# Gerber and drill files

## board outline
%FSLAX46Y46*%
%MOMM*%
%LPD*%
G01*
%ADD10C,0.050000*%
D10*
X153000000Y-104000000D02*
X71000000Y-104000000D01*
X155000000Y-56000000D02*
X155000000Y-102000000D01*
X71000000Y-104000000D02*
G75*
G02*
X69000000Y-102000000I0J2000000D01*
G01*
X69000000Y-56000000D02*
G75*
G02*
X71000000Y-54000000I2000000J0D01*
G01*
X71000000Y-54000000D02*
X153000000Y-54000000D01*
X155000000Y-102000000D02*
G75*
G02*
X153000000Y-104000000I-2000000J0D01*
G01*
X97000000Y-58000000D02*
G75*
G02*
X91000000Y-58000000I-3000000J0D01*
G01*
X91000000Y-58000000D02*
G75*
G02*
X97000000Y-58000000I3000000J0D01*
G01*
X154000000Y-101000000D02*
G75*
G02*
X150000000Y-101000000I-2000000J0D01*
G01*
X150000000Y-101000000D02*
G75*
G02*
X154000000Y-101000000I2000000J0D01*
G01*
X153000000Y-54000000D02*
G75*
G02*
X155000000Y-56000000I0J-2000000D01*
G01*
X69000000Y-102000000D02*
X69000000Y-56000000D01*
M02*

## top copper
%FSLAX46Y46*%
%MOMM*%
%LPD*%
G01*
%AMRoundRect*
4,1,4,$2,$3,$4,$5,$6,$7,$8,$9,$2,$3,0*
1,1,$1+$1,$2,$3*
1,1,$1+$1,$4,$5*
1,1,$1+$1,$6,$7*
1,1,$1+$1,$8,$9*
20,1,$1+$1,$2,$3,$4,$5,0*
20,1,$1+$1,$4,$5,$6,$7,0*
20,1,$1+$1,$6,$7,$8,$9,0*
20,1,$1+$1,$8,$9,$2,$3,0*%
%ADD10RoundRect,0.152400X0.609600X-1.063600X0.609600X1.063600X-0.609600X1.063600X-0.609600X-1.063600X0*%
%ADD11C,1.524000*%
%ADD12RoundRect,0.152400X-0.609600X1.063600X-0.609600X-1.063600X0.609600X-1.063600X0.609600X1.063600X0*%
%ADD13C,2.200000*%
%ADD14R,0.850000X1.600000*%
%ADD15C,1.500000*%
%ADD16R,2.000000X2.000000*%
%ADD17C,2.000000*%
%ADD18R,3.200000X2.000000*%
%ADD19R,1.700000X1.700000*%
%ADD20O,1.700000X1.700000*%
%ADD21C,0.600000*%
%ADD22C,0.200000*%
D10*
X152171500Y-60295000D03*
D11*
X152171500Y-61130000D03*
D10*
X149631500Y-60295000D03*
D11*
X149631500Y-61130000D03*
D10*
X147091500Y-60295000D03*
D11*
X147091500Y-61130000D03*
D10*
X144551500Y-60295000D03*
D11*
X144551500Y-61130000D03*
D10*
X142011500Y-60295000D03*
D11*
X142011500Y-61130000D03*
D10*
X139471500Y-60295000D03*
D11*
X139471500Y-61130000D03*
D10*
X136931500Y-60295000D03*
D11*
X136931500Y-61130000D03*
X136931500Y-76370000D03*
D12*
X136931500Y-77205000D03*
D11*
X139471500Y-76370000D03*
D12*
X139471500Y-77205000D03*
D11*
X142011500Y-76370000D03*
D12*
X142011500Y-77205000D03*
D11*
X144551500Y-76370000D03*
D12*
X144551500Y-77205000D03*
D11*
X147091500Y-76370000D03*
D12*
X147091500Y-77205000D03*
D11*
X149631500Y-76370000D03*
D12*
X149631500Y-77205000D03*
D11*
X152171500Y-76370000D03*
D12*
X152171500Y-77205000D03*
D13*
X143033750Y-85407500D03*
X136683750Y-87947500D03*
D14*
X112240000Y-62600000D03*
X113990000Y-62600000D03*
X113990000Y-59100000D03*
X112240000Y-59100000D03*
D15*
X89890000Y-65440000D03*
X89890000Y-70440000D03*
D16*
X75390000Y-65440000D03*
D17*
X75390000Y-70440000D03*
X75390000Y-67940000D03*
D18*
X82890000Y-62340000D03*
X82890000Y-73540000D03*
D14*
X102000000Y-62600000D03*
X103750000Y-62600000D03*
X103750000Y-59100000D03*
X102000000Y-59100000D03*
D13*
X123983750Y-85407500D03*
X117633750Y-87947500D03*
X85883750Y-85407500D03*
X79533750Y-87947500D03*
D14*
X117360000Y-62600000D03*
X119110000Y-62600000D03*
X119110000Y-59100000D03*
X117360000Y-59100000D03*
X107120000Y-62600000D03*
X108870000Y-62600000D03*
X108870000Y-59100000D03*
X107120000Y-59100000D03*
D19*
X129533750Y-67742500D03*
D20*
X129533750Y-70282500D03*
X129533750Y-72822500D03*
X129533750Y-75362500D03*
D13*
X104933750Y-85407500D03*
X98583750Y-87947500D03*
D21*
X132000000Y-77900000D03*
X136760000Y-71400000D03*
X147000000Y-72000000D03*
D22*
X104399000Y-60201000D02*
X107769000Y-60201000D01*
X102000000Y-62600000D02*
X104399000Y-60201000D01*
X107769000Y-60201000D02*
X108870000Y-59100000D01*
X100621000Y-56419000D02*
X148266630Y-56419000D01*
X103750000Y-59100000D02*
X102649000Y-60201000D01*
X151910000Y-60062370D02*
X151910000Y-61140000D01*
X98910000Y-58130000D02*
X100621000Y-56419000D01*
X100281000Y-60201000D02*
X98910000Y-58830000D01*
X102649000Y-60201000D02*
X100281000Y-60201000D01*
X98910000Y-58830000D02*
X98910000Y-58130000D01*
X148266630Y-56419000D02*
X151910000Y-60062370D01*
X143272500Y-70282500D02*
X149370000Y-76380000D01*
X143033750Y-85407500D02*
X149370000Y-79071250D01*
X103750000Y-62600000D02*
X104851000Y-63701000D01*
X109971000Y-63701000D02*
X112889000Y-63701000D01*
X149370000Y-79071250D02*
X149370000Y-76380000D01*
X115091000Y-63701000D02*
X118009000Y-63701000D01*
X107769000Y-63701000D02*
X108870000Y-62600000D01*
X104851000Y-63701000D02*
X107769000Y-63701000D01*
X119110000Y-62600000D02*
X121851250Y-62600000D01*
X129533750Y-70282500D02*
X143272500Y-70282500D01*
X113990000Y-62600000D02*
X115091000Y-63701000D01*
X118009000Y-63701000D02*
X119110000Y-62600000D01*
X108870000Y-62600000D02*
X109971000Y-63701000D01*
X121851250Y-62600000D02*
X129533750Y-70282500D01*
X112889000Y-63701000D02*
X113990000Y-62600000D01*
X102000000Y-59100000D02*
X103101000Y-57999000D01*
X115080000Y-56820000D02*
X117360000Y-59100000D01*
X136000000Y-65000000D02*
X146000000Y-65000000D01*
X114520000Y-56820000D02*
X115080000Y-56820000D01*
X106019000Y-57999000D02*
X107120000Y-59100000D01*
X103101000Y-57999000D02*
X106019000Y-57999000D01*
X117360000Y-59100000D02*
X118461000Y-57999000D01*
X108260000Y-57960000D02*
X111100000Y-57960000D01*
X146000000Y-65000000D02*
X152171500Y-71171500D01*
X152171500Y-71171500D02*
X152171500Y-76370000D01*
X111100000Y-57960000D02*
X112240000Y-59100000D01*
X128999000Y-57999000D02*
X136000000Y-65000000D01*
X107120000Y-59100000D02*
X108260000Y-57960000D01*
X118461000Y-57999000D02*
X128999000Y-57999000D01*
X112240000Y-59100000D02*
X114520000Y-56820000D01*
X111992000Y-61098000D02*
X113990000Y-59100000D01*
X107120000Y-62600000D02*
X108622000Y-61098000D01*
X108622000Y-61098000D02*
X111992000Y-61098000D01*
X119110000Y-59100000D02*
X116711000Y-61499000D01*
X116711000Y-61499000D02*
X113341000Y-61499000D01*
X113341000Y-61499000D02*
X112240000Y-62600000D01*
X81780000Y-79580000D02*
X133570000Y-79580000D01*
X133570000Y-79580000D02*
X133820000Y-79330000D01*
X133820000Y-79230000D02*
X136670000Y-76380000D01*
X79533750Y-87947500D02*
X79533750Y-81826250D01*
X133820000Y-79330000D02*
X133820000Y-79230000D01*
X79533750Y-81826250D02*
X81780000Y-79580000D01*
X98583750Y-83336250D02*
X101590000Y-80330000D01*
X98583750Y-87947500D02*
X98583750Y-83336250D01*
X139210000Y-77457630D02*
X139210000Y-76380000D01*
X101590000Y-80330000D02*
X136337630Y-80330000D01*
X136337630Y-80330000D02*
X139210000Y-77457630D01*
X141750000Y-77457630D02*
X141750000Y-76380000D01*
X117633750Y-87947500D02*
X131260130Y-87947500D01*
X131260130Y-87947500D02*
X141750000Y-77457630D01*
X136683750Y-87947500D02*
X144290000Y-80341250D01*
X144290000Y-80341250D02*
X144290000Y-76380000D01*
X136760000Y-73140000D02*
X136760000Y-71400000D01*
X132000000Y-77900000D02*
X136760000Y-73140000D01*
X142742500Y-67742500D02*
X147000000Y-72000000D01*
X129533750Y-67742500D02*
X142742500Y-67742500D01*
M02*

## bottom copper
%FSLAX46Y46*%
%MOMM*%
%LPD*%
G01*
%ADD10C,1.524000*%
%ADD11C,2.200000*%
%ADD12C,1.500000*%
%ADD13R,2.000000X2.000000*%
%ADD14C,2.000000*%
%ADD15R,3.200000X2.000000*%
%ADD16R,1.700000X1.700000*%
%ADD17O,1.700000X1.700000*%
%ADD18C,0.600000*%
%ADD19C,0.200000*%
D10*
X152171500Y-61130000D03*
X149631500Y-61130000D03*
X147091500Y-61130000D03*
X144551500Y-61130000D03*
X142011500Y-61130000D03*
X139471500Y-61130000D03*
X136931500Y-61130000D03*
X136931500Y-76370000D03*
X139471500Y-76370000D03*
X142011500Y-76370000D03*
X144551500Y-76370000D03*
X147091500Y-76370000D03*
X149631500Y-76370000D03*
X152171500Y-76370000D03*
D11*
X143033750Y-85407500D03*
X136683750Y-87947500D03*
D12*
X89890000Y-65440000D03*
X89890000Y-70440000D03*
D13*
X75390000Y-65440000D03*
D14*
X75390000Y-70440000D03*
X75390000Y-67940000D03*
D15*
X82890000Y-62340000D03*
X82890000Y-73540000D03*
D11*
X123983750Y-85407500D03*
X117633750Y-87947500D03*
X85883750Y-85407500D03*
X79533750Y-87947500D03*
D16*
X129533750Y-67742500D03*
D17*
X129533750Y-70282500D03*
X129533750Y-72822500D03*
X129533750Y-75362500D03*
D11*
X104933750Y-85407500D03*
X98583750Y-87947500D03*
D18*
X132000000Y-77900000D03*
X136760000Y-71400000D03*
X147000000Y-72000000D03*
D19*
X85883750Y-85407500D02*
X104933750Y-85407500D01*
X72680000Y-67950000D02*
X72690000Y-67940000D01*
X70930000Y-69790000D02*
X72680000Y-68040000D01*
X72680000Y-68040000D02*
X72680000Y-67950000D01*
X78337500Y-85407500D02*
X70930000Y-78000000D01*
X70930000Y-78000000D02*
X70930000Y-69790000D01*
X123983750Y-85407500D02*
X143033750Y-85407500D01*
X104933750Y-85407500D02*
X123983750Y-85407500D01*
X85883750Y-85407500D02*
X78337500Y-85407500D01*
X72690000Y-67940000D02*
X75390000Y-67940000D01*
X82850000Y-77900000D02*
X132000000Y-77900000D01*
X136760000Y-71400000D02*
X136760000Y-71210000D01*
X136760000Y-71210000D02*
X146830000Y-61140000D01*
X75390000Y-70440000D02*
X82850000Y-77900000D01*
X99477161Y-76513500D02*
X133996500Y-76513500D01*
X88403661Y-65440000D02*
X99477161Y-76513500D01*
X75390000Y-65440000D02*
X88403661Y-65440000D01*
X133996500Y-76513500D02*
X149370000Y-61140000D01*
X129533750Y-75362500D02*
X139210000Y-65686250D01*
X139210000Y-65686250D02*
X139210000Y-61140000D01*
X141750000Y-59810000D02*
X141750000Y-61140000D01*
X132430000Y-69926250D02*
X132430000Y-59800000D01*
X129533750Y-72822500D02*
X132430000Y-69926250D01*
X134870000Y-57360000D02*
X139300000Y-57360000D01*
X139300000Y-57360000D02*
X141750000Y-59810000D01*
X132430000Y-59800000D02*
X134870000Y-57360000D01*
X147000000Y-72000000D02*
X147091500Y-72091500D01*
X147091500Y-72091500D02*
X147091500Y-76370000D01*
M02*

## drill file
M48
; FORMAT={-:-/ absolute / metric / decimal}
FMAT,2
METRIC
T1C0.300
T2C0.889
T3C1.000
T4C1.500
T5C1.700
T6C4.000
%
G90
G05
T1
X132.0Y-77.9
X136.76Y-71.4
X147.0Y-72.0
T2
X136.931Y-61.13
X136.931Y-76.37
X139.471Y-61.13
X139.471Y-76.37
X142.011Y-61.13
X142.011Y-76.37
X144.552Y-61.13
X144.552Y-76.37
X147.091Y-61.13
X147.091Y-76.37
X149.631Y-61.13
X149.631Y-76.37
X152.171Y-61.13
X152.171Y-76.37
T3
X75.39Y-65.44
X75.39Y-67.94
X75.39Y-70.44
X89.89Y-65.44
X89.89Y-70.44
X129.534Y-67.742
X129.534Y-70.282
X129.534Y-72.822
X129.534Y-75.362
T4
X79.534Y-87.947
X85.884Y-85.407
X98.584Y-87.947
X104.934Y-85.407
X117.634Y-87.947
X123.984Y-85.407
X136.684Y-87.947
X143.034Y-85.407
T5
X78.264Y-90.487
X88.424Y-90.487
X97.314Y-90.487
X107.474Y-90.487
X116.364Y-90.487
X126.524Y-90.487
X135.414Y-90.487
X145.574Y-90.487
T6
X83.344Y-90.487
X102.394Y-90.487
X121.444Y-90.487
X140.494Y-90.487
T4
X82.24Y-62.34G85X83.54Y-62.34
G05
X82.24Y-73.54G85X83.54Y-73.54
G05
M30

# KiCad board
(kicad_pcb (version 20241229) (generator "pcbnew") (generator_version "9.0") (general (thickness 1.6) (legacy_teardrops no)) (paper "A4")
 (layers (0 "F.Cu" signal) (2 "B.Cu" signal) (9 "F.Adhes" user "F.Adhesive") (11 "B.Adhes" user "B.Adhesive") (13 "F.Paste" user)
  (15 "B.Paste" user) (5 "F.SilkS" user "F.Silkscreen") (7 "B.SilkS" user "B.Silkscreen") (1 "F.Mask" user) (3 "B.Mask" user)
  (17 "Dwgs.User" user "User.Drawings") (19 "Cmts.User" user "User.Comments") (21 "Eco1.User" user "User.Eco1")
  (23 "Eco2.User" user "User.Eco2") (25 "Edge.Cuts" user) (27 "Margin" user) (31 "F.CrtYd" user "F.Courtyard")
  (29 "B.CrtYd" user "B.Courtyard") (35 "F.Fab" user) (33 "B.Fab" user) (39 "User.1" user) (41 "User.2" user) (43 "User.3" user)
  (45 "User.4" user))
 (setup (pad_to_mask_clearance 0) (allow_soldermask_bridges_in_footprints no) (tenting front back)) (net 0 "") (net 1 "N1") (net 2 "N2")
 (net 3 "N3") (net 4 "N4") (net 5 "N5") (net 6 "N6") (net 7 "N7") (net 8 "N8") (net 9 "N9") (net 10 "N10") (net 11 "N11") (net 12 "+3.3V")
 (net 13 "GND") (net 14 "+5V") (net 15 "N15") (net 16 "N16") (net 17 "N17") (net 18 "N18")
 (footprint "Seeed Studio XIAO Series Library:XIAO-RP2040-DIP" (layer "F.Cu") (at 144.5515 68.75 -90)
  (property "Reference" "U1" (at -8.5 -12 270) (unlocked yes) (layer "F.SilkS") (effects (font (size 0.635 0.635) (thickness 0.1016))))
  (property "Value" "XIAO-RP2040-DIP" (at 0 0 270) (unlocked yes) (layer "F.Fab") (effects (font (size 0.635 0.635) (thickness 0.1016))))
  (pad "1" smd roundrect (at -8.455 -7.62 90) (size 2.432 1.524) (layers "F.Cu" "F.Mask") (roundrect_rratio 0.1) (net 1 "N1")
   (thermal_bridge_angle 45))
  (pad "1" thru_hole circle (at -7.62 -7.62 90) (size 1.524 1.524) (drill 0.889) (layers "*.Cu" "*.Mask") (remove_unused_layers no)
   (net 1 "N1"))
  (pad "2" smd roundrect (at -8.455 -5.08 90) (size 2.432 1.524) (layers "F.Cu" "F.Mask") (roundrect_rratio 0.1) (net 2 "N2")
   (thermal_bridge_angle 45))
  (pad "2" thru_hole circle (at -7.62 -5.08 90) (size 1.524 1.524) (drill 0.889) (layers "*.Cu" "*.Mask") (remove_unused_layers no)
   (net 2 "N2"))
  (pad "3" smd roundrect (at -8.455 -2.54 90) (size 2.432 1.524) (layers "F.Cu" "F.Mask") (roundrect_rratio 0.1) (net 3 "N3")
   (thermal_bridge_angle 45))
  (pad "3" thru_hole circle (at -7.62 -2.54 90) (size 1.524 1.524) (drill 0.889) (layers "*.Cu" "*.Mask") (remove_unused_layers no)
   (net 3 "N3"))
  (pad "4" smd roundrect (at -8.455 0 90) (size 2.432 1.524) (layers "F.Cu" "F.Mask") (roundrect_rratio 0.1) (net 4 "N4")
   (thermal_bridge_angle 45))
  (pad "4" thru_hole circle (at -7.62 0 90) (size 1.524 1.524) (drill 0.889) (layers "*.Cu" "*.Mask") (remove_unused_layers no) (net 4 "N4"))
  (pad "5" smd roundrect (at -8.455 2.54 90) (size 2.432 1.524) (layers "F.Cu" "F.Mask") (roundrect_rratio 0.1) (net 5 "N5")
   (thermal_bridge_angle 45))
  (pad "5" thru_hole circle (at -7.62 2.54 90) (size 1.524 1.524) (drill 0.889) (layers "*.Cu" "*.Mask") (remove_unused_layers no)
   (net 5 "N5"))
  (pad "6" smd roundrect (at -8.455 5.08 90) (size 2.432 1.524) (layers "F.Cu" "F.Mask") (roundrect_rratio 0.1) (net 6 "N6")
   (thermal_bridge_angle 45))
  (pad "6" thru_hole circle (at -7.62 5.08 90) (size 1.524 1.524) (drill 0.889) (layers "*.Cu" "*.Mask") (remove_unused_layers no)
   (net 6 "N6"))
  (pad "7" smd roundrect (at -8.455 7.62 90) (size 2.432 1.524) (layers "F.Cu" "F.Mask") (roundrect_rratio 0.1) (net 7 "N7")
   (thermal_bridge_angle 45))
  (pad "7" thru_hole circle (at -7.62 7.62 90) (size 1.524 1.524) (drill 0.889) (layers "*.Cu" "*.Mask") (remove_unused_layers no)
   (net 7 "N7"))
  (pad "8" thru_hole circle (at 7.62 7.62 270) (size 1.524 1.524) (drill 0.889) (layers "*.Cu" "*.Mask") (remove_unused_layers no)
   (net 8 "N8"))
  (pad "8" smd roundrect (at 8.455 7.62 270) (size 2.432 1.524) (layers "F.Cu" "F.Mask") (roundrect_rratio 0.1) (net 8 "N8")
   (thermal_bridge_angle 45))
  (pad "9" thru_hole circle (at 7.62 5.08 270) (size 1.524 1.524) (drill 0.889) (layers "*.Cu" "*.Mask") (remove_unused_layers no)
   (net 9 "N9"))
  (pad "9" smd roundrect (at 8.455 5.08 270) (size 2.432 1.524) (layers "F.Cu" "F.Mask") (roundrect_rratio 0.1) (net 9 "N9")
   (thermal_bridge_angle 45))
  (pad "10" thru_hole circle (at 7.62 2.54 270) (size 1.524 1.524) (drill 0.889) (layers "*.Cu" "*.Mask") (remove_unused_layers no)
   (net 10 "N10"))
  (pad "10" smd roundrect (at 8.455 2.54 270) (size 2.432 1.524) (layers "F.Cu" "F.Mask") (roundrect_rratio 0.1) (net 10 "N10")
   (thermal_bridge_angle 45))
  (pad "11" thru_hole circle (at 7.62 0 270) (size 1.524 1.524) (drill 0.889) (layers "*.Cu" "*.Mask") (remove_unused_layers no)
   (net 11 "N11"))
  (pad "11" smd roundrect (at 8.455 0 270) (size 2.432 1.524) (layers "F.Cu" "F.Mask") (roundrect_rratio 0.1) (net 11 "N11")
   (thermal_bridge_angle 45))
  (pad "12" thru_hole circle (at 7.62 -2.54 270) (size 1.524 1.524) (drill 0.889) (layers "*.Cu" "*.Mask") (remove_unused_layers no)
   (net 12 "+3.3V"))
  (pad "12" smd roundrect (at 8.455 -2.54 270) (size 2.432 1.524) (layers "F.Cu" "F.Mask") (roundrect_rratio 0.1) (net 12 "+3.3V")
   (thermal_bridge_angle 45))
  (pad "13" thru_hole circle (at 7.62 -5.08 270) (size 1.524 1.524) (drill 0.889) (layers "*.Cu" "*.Mask") (remove_unused_layers no)
   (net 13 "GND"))
  (pad "13" smd roundrect (at 8.455 -5.08 270) (size 2.432 1.524) (layers "F.Cu" "F.Mask") (roundrect_rratio 0.1) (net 13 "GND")
   (thermal_bridge_angle 45))
  (pad "14" thru_hole circle (at 7.62 -7.62 270) (size 1.524 1.524) (drill 0.889) (layers "*.Cu" "*.Mask") (remove_unused_layers no)
   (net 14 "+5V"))
  (pad "14" smd roundrect (at 8.455 -7.62 270) (size 2.432 1.524) (layers "F.Cu" "F.Mask") (roundrect_rratio 0.1) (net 14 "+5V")
   (thermal_bridge_angle 45)))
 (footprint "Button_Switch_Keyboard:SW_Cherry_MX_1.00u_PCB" (layer "F.Cu") (at 143.03375 85.4075)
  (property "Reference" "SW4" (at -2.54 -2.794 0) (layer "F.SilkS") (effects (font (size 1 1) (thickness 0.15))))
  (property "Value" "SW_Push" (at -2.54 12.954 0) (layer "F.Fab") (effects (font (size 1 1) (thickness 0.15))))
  (pad "" np_thru_hole circle (at -7.62 5.08) (size 1.7 1.7) (drill 1.7) (layers "*.Cu" "*.Mask"))
  (pad "" np_thru_hole circle (at -2.54 5.08) (size 4 4) (drill 4) (layers "*.Cu" "*.Mask"))
  (pad "" np_thru_hole circle (at 2.54 5.08) (size 1.7 1.7) (drill 1.7) (layers "*.Cu" "*.Mask"))
  (pad "1" thru_hole circle (at 0 0) (size 2.2 2.2) (drill 1.5) (layers "*.Cu" "*.Mask") (remove_unused_layers no) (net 13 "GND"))
  (pad "2" thru_hole circle (at -6.35 2.54) (size 2.2 2.2) (drill 1.5) (layers "*.Cu" "*.Mask") (remove_unused_layers no) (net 11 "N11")))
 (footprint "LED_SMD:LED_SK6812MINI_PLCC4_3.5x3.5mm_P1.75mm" (layer "F.Cu") (at 113.115 60.85 90)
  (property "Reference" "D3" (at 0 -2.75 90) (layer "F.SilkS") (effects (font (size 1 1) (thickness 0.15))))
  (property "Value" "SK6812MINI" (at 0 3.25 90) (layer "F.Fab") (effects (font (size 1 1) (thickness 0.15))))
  (pad "1" smd rect (at -1.75 -0.875 90) (size 1.6 0.85) (layers "F.Cu" "F.Mask" "F.Paste") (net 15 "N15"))
  (pad "2" smd rect (at -1.75 0.875 90) (size 1.6 0.85) (layers "F.Cu" "F.Mask" "F.Paste") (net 13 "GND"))
  (pad "3" smd rect (at 1.75 0.875 90) (size 1.6 0.85) (layers "F.Cu" "F.Mask" "F.Paste") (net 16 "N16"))
  (pad "4" smd rect (at 1.75 -0.875 90) (size 1.6 0.85) (layers "F.Cu" "F.Mask" "F.Paste") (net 14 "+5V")))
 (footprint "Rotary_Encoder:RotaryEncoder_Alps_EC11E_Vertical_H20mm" (layer "F.Cu") (at 75.39 65.44)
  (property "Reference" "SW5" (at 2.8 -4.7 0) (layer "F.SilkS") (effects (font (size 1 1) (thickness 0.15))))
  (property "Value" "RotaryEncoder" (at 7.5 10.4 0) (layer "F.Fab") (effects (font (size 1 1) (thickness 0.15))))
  (pad "" thru_hole circle (at 14.5 0) (size 1.5 1.5) (drill 1) (layers "*.Cu" "*.Mask") (remove_unused_layers no))
  (pad "" thru_hole circle (at 14.5 5) (size 1.5 1.5) (drill 1) (layers "*.Cu" "*.Mask") (remove_unused_layers no))
  (pad "A" thru_hole rect (at 0 0) (size 2 2) (drill 1) (layers "*.Cu" "*.Mask") (remove_unused_layers no) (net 2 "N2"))
  (pad "B" thru_hole circle (at 0 5) (size 2 2) (drill 1) (layers "*.Cu" "*.Mask") (remove_unused_layers no) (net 3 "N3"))
  (pad "C" thru_hole circle (at 0 2.5) (size 2 2) (drill 1) (layers "*.Cu" "*.Mask") (remove_unused_layers no) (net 13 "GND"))
  (pad "MP" thru_hole rect (at 7.5 -3.1) (size 3.2 2) (drill oval 2.8 1.5) (layers "*.Cu" "*.Mask") (remove_unused_layers no))
  (pad "MP" thru_hole rect (at 7.5 8.1) (size 3.2 2) (drill oval 2.8 1.5) (layers "*.Cu" "*.Mask") (remove_unused_layers no)))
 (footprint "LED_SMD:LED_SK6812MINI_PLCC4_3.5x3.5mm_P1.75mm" (layer "F.Cu") (at 102.875 60.85 90)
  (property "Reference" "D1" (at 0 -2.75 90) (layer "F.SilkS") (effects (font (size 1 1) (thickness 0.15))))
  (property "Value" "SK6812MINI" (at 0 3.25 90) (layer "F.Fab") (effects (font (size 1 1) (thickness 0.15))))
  (pad "1" smd rect (at -1.75 -0.875 90) (size 1.6 0.85) (layers "F.Cu" "F.Mask" "F.Paste") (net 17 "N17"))
  (pad "2" smd rect (at -1.75 0.875 90) (size 1.6 0.85) (layers "F.Cu" "F.Mask" "F.Paste") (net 13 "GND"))
  (pad "3" smd rect (at 1.75 0.875 90) (size 1.6 0.85) (layers "F.Cu" "F.Mask" "F.Paste") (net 1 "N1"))
  (pad "4" smd rect (at 1.75 -0.875 90) (size 1.6 0.85) (layers "F.Cu" "F.Mask" "F.Paste") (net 14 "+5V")))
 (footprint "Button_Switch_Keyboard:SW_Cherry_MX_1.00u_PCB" (layer "F.Cu") (at 123.98375 85.4075)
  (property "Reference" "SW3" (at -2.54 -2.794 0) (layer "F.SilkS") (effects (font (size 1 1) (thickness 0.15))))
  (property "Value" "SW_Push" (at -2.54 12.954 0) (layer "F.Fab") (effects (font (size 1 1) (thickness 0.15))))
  (pad "" np_thru_hole circle (at -7.62 5.08) (size 1.7 1.7) (drill 1.7) (layers "*.Cu" "*.Mask"))
  (pad "" np_thru_hole circle (at -2.54 5.08) (size 4 4) (drill 4) (layers "*.Cu" "*.Mask"))
  (pad "" np_thru_hole circle (at 2.54 5.08) (size 1.7 1.7) (drill 1.7) (layers "*.Cu" "*.Mask"))
  (pad "1" thru_hole circle (at 0 0) (size 2.2 2.2) (drill 1.5) (layers "*.Cu" "*.Mask") (remove_unused_layers no) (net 13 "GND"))
  (pad "2" thru_hole circle (at -6.35 2.54) (size 2.2 2.2) (drill 1.5) (layers "*.Cu" "*.Mask") (remove_unused_layers no) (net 10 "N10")))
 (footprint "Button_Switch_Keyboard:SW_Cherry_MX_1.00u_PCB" (layer "F.Cu") (at 85.88375 85.4075)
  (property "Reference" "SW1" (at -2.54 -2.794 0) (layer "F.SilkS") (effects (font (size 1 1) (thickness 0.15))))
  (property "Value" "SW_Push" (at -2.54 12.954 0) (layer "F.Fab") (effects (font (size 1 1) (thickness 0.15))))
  (pad "" np_thru_hole circle (at -7.62 5.08) (size 1.7 1.7) (drill 1.7) (layers "*.Cu" "*.Mask"))
  (pad "" np_thru_hole circle (at -2.54 5.08) (size 4 4) (drill 4) (layers "*.Cu" "*.Mask"))
  (pad "" np_thru_hole circle (at 2.54 5.08) (size 1.7 1.7) (drill 1.7) (layers "*.Cu" "*.Mask"))
  (pad "1" thru_hole circle (at 0 0) (size 2.2 2.2) (drill 1.5) (layers "*.Cu" "*.Mask") (remove_unused_layers no) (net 13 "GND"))
  (pad "2" thru_hole circle (at -6.35 2.54) (size 2.2 2.2) (drill 1.5) (layers "*.Cu" "*.Mask") (remove_unused_layers no) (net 8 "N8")))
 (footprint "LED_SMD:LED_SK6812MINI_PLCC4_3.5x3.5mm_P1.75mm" (layer "F.Cu") (at 118.235 60.85 90)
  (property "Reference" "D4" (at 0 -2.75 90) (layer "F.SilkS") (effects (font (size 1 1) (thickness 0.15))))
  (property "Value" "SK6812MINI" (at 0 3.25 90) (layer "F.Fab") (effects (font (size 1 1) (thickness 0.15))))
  (pad "1" smd rect (at -1.75 -0.875 90) (size 1.6 0.85) (layers "F.Cu" "F.Mask" "F.Paste") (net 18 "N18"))
  (pad "2" smd rect (at -1.75 0.875 90) (size 1.6 0.85) (layers "F.Cu" "F.Mask" "F.Paste") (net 13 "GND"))
  (pad "3" smd rect (at 1.75 0.875 90) (size 1.6 0.85) (layers "F.Cu" "F.Mask" "F.Paste") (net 15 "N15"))
  (pad "4" smd rect (at 1.75 -0.875 90) (size 1.6 0.85) (layers "F.Cu" "F.Mask" "F.Paste") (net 14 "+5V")))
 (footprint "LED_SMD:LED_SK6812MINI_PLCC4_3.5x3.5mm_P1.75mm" (layer "F.Cu") (at 107.995 60.85 90)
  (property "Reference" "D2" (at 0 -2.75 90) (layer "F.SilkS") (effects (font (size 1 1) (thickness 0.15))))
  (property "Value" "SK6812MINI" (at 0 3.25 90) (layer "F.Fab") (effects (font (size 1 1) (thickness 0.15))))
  (pad "1" smd rect (at -1.75 -0.875 90) (size 1.6 0.85) (layers "F.Cu" "F.Mask" "F.Paste") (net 16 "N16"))
  (pad "2" smd rect (at -1.75 0.875 90) (size 1.6 0.85) (layers "F.Cu" "F.Mask" "F.Paste") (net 13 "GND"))
  (pad "3" smd rect (at 1.75 0.875 90) (size 1.6 0.85) (layers "F.Cu" "F.Mask" "F.Paste") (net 17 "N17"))
  (pad "4" smd rect (at 1.75 -0.875 90) (size 1.6 0.85) (layers "F.Cu" "F.Mask" "F.Paste") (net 14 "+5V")))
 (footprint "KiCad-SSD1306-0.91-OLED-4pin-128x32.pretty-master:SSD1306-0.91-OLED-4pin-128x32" (layer "F.Cu") (at 93.03375 65.5525)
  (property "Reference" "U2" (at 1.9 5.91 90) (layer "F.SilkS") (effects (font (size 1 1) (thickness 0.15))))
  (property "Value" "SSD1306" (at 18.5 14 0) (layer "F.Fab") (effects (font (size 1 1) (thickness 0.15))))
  (pad "1" thru_hole rect (at 36.5 2.19) (size 1.7 1.7) (drill 1) (layers "*.Cu" "*.Mask") (remove_unused_layers no) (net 12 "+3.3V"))
  (pad "2" thru_hole oval (at 36.5 4.73) (size 1.7 1.7) (drill 1) (layers "*.Cu" "*.Mask") (remove_unused_layers no) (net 13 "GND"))
  (pad "3" thru_hole oval (at 36.5 7.27) (size 1.7 1.7) (drill 1) (layers "*.Cu" "*.Mask") (remove_unused_layers no) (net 5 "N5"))
  (pad "4" thru_hole oval (at 36.5 9.81) (size 1.7 1.7) (drill 1) (layers "*.Cu" "*.Mask") (remove_unused_layers no) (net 6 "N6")))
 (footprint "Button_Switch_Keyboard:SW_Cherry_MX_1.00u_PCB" (layer "F.Cu") (at 104.93375 85.4075)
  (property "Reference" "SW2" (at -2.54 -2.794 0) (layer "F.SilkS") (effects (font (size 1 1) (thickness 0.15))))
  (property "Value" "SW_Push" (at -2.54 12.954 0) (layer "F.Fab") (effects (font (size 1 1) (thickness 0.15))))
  (pad "" np_thru_hole circle (at -7.62 5.08) (size 1.7 1.7) (drill 1.7) (layers "*.Cu" "*.Mask"))
  (pad "" np_thru_hole circle (at -2.54 5.08) (size 4 4) (drill 4) (layers "*.Cu" "*.Mask"))
  (pad "" np_thru_hole circle (at 2.54 5.08) (size 1.7 1.7) (drill 1.7) (layers "*.Cu" "*.Mask"))
  (pad "1" thru_hole circle (at 0 0) (size 2.2 2.2) (drill 1.5) (layers "*.Cu" "*.Mask") (remove_unused_layers no) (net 13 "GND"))
  (pad "2" thru_hole circle (at -6.35 2.54) (size 2.2 2.2) (drill 1.5) (layers "*.Cu" "*.Mask") (remove_unused_layers no) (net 9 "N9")))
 (gr_line (start 153 104) (end 71 104) (stroke (width 0.05) (type default)) (layer "Edge.Cuts"))
 (gr_line (start 155 56) (end 155 102) (stroke (width 0.05) (type default)) (layer "Edge.Cuts"))
 (gr_arc (start 71 104) (mid 69.585786 103.414214) (end 69 102) (stroke (width 0.05) (type default)) (layer "Edge.Cuts"))
 (gr_arc (start 69 56) (mid 69.585786 54.585786) (end 71 54) (stroke (width 0.05) (type default)) (layer "Edge.Cuts"))
 (gr_line (start 71 54) (end 153 54) (stroke (width 0.05) (type default)) (layer "Edge.Cuts"))
 (gr_arc (start 155 102) (mid 154.414214 103.414214) (end 153 104) (stroke (width 0.05) (type default)) (layer "Edge.Cuts"))
 (gr_circle (center 94 58) (end 97 58) (stroke (width 0.05) (type default)) (fill no) (layer "Edge.Cuts"))
 (gr_circle (center 152 101) (end 152 99) (stroke (width 0.05) (type default)) (fill no) (layer "Edge.Cuts"))
 (gr_arc (start 153 54) (mid 154.414214 54.585786) (end 155 56) (stroke (width 0.05) (type default)) (layer "Edge.Cuts"))
 (gr_line (start 69 102) (end 69 56) (stroke (width 0.05) (type default)) (layer "Edge.Cuts"))
 (segment (start 104.399 60.201) (end 107.769 60.201) (width 0.2) (layer "F.Cu") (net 17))
 (segment (start 102 62.6) (end 104.399 60.201) (width 0.2) (layer "F.Cu") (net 17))
 (segment (start 107.769 60.201) (end 108.87 59.1) (width 0.2) (layer "F.Cu") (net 17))
 (segment (start 100.621 56.419) (end 148.26663 56.419) (width 0.2) (layer "F.Cu") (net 1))
 (segment (start 103.75 59.1) (end 102.649 60.201) (width 0.2) (layer "F.Cu") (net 1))
 (segment (start 151.91 60.06237) (end 151.91 61.14) (width 0.2) (layer "F.Cu") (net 1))
 (segment (start 98.91 58.13) (end 100.621 56.419) (width 0.2) (layer "F.Cu") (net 1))
 (segment (start 100.281 60.201) (end 98.91 58.83) (width 0.2) (layer "F.Cu") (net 1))
 (segment (start 102.649 60.201) (end 100.281 60.201) (width 0.2) (layer "F.Cu") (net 1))
 (segment (start 98.91 58.83) (end 98.91 58.13) (width 0.2) (layer "F.Cu") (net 1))
 (segment (start 148.26663 56.419) (end 151.91 60.06237) (width 0.2) (layer "F.Cu") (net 1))
 (segment (start 143.2725 70.2825) (end 149.37 76.38) (width 0.2) (layer "F.Cu") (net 13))
 (segment (start 143.03375 85.4075) (end 149.37 79.07125) (width 0.2) (layer "F.Cu") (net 13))
 (segment (start 103.75 62.6) (end 104.851 63.701) (width 0.2) (layer "F.Cu") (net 13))
 (segment (start 109.971 63.701) (end 112.889 63.701) (width 0.2) (layer "F.Cu") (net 13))
 (segment (start 149.37 79.07125) (end 149.37 76.38) (width 0.2) (layer "F.Cu") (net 13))
 (segment (start 115.091 63.701) (end 118.009 63.701) (width 0.2) (layer "F.Cu") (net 13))
 (segment (start 107.769 63.701) (end 108.87 62.6) (width 0.2) (layer "F.Cu") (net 13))
 (segment (start 104.851 63.701) (end 107.769 63.701) (width 0.2) (layer "F.Cu") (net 13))
 (segment (start 119.11 62.6) (end 121.85125 62.6) (width 0.2) (layer "F.Cu") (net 13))
 (segment (start 129.53375 70.2825) (end 143.2725 70.2825) (width 0.2) (layer "F.Cu") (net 13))
 (segment (start 113.99 62.6) (end 115.091 63.701) (width 0.2) (layer "F.Cu") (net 13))
 (segment (start 118.009 63.701) (end 119.11 62.6) (width 0.2) (layer "F.Cu") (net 13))
 (segment (start 108.87 62.6) (end 109.971 63.701) (width 0.2) (layer "F.Cu") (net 13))
 (segment (start 121.85125 62.6) (end 129.53375 70.2825) (width 0.2) (layer "F.Cu") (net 13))
 (segment (start 112.889 63.701) (end 113.99 62.6) (width 0.2) (layer "F.Cu") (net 13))
 (segment (start 85.88375 85.4075) (end 104.93375 85.4075) (width 0.2) (layer "B.Cu") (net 13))
 (segment (start 72.68 67.95) (end 72.69 67.94) (width 0.2) (layer "B.Cu") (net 13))
 (segment (start 70.93 69.79) (end 72.68 68.04) (width 0.2) (layer "B.Cu") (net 13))
 (segment (start 72.68 68.04) (end 72.68 67.95) (width 0.2) (layer "B.Cu") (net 13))
 (segment (start 78.3375 85.4075) (end 70.93 78) (width 0.2) (layer "B.Cu") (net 13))
 (segment (start 70.93 78) (end 70.93 69.79) (width 0.2) (layer "B.Cu") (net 13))
 (segment (start 123.98375 85.4075) (end 143.03375 85.4075) (width 0.2) (layer "B.Cu") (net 13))
 (segment (start 104.93375 85.4075) (end 123.98375 85.4075) (width 0.2) (layer "B.Cu") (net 13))
 (segment (start 85.88375 85.4075) (end 78.3375 85.4075) (width 0.2) (layer "B.Cu") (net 13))
 (segment (start 72.69 67.94) (end 75.39 67.94) (width 0.2) (layer "B.Cu") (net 13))
 (segment (start 102 59.1) (end 103.101 57.999) (width 0.2) (layer "F.Cu") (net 14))
 (segment (start 115.08 56.82) (end 117.36 59.1) (width 0.2) (layer "F.Cu") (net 14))
 (segment (start 136 65) (end 146 65) (width 0.2) (layer "F.Cu") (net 14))
 (segment (start 114.52 56.82) (end 115.08 56.82) (width 0.2) (layer "F.Cu") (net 14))
 (segment (start 106.019 57.999) (end 107.12 59.1) (width 0.2) (layer "F.Cu") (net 14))
 (segment (start 103.101 57.999) (end 106.019 57.999) (width 0.2) (layer "F.Cu") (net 14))
 (segment (start 117.36 59.1) (end 118.461 57.999) (width 0.2) (layer "F.Cu") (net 14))
 (segment (start 108.26 57.96) (end 111.1 57.96) (width 0.2) (layer "F.Cu") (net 14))
 (segment (start 146 65) (end 152.1715 71.1715) (width 0.2) (layer "F.Cu") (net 14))
 (segment (start 152.1715 71.1715) (end 152.1715 76.37) (width 0.2) (layer "F.Cu") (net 14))
 (segment (start 111.1 57.96) (end 112.24 59.1) (width 0.2) (layer "F.Cu") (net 14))
 (segment (start 128.999 57.999) (end 136 65) (width 0.2) (layer "F.Cu") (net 14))
 (segment (start 107.12 59.1) (end 108.26 57.96) (width 0.2) (layer "F.Cu") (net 14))
 (segment (start 118.461 57.999) (end 128.999 57.999) (width 0.2) (layer "F.Cu") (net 14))
 (segment (start 112.24 59.1) (end 114.52 56.82) (width 0.2) (layer "F.Cu") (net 14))
 (segment (start 111.992 61.098) (end 113.99 59.1) (width 0.2) (layer "F.Cu") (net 16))
 (segment (start 107.12 62.6) (end 108.622 61.098) (width 0.2) (layer "F.Cu") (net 16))
 (segment (start 108.622 61.098) (end 111.992 61.098) (width 0.2) (layer "F.Cu") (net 16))
 (segment (start 119.11 59.1) (end 116.711 61.499) (width 0.2) (layer "F.Cu") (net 15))
 (segment (start 116.711 61.499) (end 113.341 61.499) (width 0.2) (layer "F.Cu") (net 15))
 (segment (start 113.341 61.499) (end 112.24 62.6) (width 0.2) (layer "F.Cu") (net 15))
 (segment (start 81.78 79.58) (end 133.57 79.58) (width 0.2) (layer "F.Cu") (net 8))
 (segment (start 133.57 79.58) (end 133.82 79.33) (width 0.2) (layer "F.Cu") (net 8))
 (segment (start 133.82 79.23) (end 136.67 76.38) (width 0.2) (layer "F.Cu") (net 8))
 (segment (start 79.53375 87.9475) (end 79.53375 81.82625) (width 0.2) (layer "F.Cu") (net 8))
 (segment (start 133.82 79.33) (end 133.82 79.23) (width 0.2) (layer "F.Cu") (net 8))
 (segment (start 79.53375 81.82625) (end 81.78 79.58) (width 0.2) (layer "F.Cu") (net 8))
 (segment (start 98.58375 83.33625) (end 101.59 80.33) (width 0.2) (layer "F.Cu") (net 9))
 (segment (start 98.58375 87.9475) (end 98.58375 83.33625) (width 0.2) (layer "F.Cu") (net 9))
 (segment (start 139.21 77.45763) (end 139.21 76.38) (width 0.2) (layer "F.Cu") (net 9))
 (segment (start 101.59 80.33) (end 136.33763 80.33) (width 0.2) (layer "F.Cu") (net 9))
 (segment (start 136.33763 80.33) (end 139.21 77.45763) (width 0.2) (layer "F.Cu") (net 9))
 (segment (start 141.75 77.45763) (end 141.75 76.38) (width 0.2) (layer "F.Cu") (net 10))
 (segment (start 117.63375 87.9475) (end 131.26013 87.9475) (width 0.2) (layer "F.Cu") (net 10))
 (segment (start 131.26013 87.9475) (end 141.75 77.45763) (width 0.2) (layer "F.Cu") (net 10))
 (segment (start 136.68375 87.9475) (end 144.29 80.34125) (width 0.2) (layer "F.Cu") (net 11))
 (segment (start 144.29 80.34125) (end 144.29 76.38) (width 0.2) (layer "F.Cu") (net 11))
 (segment (start 136.76 73.14) (end 136.76 71.4) (width 0.2) (layer "F.Cu") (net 3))
 (segment (start 132 77.9) (end 136.76 73.14) (width 0.2) (layer "F.Cu") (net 3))
 (via (at 132 77.9) (size 0.6) (drill 0.3) (layers "F.Cu" "B.Cu") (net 3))
 (via (at 136.76 71.4) (size 0.6) (drill 0.3) (layers "F.Cu" "B.Cu") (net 3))
 (segment (start 82.85 77.9) (end 132 77.9) (width 0.2) (layer "B.Cu") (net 3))
 (segment (start 136.76 71.4) (end 136.76 71.21) (width 0.2) (layer "B.Cu") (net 3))
 (segment (start 136.76 71.21) (end 146.83 61.14) (width 0.2) (layer "B.Cu") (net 3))
 (segment (start 75.39 70.44) (end 82.85 77.9) (width 0.2) (layer "B.Cu") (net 3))
 (segment (start 99.477161 76.5135) (end 133.9965 76.5135) (width 0.2) (layer "B.Cu") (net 2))
 (segment (start 88.403661 65.44) (end 99.477161 76.5135) (width 0.2) (layer "B.Cu") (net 2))
 (segment (start 75.39 65.44) (end 88.403661 65.44) (width 0.2) (layer "B.Cu") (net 2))
 (segment (start 133.9965 76.5135) (end 149.37 61.14) (width 0.2) (layer "B.Cu") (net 2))
 (segment (start 129.53375 75.3625) (end 139.21 65.68625) (width 0.2) (layer "B.Cu") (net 6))
 (segment (start 139.21 65.68625) (end 139.21 61.14) (width 0.2) (layer "B.Cu") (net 6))
 (segment (start 141.75 59.81) (end 141.75 61.14) (width 0.2) (layer "B.Cu") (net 5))
 (segment (start 132.43 69.92625) (end 132.43 59.8) (width 0.2) (layer "B.Cu") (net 5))
 (segment (start 129.53375 72.8225) (end 132.43 69.92625) (width 0.2) (layer "B.Cu") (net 5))
 (segment (start 134.87 57.36) (end 139.3 57.36) (width 0.2) (layer "B.Cu") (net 5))
 (segment (start 139.3 57.36) (end 141.75 59.81) (width 0.2) (layer "B.Cu") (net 5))
 (segment (start 132.43 59.8) (end 134.87 57.36) (width 0.2) (layer "B.Cu") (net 5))
 (segment (start 142.7425 67.7425) (end 147 72) (width 0.2) (layer "F.Cu") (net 12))
 (segment (start 129.53375 67.7425) (end 142.7425 67.7425) (width 0.2) (layer "F.Cu") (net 12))
 (via (at 147 72) (size 0.6) (drill 0.3) (layers "F.Cu" "B.Cu") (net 12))
 (segment (start 147 72) (end 147.0915 72.0915) (width 0.2) (layer "B.Cu") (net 12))
 (segment (start 147.0915 72.0915) (end 147.0915 76.37) (width 0.2) (layer "B.Cu") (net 12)))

